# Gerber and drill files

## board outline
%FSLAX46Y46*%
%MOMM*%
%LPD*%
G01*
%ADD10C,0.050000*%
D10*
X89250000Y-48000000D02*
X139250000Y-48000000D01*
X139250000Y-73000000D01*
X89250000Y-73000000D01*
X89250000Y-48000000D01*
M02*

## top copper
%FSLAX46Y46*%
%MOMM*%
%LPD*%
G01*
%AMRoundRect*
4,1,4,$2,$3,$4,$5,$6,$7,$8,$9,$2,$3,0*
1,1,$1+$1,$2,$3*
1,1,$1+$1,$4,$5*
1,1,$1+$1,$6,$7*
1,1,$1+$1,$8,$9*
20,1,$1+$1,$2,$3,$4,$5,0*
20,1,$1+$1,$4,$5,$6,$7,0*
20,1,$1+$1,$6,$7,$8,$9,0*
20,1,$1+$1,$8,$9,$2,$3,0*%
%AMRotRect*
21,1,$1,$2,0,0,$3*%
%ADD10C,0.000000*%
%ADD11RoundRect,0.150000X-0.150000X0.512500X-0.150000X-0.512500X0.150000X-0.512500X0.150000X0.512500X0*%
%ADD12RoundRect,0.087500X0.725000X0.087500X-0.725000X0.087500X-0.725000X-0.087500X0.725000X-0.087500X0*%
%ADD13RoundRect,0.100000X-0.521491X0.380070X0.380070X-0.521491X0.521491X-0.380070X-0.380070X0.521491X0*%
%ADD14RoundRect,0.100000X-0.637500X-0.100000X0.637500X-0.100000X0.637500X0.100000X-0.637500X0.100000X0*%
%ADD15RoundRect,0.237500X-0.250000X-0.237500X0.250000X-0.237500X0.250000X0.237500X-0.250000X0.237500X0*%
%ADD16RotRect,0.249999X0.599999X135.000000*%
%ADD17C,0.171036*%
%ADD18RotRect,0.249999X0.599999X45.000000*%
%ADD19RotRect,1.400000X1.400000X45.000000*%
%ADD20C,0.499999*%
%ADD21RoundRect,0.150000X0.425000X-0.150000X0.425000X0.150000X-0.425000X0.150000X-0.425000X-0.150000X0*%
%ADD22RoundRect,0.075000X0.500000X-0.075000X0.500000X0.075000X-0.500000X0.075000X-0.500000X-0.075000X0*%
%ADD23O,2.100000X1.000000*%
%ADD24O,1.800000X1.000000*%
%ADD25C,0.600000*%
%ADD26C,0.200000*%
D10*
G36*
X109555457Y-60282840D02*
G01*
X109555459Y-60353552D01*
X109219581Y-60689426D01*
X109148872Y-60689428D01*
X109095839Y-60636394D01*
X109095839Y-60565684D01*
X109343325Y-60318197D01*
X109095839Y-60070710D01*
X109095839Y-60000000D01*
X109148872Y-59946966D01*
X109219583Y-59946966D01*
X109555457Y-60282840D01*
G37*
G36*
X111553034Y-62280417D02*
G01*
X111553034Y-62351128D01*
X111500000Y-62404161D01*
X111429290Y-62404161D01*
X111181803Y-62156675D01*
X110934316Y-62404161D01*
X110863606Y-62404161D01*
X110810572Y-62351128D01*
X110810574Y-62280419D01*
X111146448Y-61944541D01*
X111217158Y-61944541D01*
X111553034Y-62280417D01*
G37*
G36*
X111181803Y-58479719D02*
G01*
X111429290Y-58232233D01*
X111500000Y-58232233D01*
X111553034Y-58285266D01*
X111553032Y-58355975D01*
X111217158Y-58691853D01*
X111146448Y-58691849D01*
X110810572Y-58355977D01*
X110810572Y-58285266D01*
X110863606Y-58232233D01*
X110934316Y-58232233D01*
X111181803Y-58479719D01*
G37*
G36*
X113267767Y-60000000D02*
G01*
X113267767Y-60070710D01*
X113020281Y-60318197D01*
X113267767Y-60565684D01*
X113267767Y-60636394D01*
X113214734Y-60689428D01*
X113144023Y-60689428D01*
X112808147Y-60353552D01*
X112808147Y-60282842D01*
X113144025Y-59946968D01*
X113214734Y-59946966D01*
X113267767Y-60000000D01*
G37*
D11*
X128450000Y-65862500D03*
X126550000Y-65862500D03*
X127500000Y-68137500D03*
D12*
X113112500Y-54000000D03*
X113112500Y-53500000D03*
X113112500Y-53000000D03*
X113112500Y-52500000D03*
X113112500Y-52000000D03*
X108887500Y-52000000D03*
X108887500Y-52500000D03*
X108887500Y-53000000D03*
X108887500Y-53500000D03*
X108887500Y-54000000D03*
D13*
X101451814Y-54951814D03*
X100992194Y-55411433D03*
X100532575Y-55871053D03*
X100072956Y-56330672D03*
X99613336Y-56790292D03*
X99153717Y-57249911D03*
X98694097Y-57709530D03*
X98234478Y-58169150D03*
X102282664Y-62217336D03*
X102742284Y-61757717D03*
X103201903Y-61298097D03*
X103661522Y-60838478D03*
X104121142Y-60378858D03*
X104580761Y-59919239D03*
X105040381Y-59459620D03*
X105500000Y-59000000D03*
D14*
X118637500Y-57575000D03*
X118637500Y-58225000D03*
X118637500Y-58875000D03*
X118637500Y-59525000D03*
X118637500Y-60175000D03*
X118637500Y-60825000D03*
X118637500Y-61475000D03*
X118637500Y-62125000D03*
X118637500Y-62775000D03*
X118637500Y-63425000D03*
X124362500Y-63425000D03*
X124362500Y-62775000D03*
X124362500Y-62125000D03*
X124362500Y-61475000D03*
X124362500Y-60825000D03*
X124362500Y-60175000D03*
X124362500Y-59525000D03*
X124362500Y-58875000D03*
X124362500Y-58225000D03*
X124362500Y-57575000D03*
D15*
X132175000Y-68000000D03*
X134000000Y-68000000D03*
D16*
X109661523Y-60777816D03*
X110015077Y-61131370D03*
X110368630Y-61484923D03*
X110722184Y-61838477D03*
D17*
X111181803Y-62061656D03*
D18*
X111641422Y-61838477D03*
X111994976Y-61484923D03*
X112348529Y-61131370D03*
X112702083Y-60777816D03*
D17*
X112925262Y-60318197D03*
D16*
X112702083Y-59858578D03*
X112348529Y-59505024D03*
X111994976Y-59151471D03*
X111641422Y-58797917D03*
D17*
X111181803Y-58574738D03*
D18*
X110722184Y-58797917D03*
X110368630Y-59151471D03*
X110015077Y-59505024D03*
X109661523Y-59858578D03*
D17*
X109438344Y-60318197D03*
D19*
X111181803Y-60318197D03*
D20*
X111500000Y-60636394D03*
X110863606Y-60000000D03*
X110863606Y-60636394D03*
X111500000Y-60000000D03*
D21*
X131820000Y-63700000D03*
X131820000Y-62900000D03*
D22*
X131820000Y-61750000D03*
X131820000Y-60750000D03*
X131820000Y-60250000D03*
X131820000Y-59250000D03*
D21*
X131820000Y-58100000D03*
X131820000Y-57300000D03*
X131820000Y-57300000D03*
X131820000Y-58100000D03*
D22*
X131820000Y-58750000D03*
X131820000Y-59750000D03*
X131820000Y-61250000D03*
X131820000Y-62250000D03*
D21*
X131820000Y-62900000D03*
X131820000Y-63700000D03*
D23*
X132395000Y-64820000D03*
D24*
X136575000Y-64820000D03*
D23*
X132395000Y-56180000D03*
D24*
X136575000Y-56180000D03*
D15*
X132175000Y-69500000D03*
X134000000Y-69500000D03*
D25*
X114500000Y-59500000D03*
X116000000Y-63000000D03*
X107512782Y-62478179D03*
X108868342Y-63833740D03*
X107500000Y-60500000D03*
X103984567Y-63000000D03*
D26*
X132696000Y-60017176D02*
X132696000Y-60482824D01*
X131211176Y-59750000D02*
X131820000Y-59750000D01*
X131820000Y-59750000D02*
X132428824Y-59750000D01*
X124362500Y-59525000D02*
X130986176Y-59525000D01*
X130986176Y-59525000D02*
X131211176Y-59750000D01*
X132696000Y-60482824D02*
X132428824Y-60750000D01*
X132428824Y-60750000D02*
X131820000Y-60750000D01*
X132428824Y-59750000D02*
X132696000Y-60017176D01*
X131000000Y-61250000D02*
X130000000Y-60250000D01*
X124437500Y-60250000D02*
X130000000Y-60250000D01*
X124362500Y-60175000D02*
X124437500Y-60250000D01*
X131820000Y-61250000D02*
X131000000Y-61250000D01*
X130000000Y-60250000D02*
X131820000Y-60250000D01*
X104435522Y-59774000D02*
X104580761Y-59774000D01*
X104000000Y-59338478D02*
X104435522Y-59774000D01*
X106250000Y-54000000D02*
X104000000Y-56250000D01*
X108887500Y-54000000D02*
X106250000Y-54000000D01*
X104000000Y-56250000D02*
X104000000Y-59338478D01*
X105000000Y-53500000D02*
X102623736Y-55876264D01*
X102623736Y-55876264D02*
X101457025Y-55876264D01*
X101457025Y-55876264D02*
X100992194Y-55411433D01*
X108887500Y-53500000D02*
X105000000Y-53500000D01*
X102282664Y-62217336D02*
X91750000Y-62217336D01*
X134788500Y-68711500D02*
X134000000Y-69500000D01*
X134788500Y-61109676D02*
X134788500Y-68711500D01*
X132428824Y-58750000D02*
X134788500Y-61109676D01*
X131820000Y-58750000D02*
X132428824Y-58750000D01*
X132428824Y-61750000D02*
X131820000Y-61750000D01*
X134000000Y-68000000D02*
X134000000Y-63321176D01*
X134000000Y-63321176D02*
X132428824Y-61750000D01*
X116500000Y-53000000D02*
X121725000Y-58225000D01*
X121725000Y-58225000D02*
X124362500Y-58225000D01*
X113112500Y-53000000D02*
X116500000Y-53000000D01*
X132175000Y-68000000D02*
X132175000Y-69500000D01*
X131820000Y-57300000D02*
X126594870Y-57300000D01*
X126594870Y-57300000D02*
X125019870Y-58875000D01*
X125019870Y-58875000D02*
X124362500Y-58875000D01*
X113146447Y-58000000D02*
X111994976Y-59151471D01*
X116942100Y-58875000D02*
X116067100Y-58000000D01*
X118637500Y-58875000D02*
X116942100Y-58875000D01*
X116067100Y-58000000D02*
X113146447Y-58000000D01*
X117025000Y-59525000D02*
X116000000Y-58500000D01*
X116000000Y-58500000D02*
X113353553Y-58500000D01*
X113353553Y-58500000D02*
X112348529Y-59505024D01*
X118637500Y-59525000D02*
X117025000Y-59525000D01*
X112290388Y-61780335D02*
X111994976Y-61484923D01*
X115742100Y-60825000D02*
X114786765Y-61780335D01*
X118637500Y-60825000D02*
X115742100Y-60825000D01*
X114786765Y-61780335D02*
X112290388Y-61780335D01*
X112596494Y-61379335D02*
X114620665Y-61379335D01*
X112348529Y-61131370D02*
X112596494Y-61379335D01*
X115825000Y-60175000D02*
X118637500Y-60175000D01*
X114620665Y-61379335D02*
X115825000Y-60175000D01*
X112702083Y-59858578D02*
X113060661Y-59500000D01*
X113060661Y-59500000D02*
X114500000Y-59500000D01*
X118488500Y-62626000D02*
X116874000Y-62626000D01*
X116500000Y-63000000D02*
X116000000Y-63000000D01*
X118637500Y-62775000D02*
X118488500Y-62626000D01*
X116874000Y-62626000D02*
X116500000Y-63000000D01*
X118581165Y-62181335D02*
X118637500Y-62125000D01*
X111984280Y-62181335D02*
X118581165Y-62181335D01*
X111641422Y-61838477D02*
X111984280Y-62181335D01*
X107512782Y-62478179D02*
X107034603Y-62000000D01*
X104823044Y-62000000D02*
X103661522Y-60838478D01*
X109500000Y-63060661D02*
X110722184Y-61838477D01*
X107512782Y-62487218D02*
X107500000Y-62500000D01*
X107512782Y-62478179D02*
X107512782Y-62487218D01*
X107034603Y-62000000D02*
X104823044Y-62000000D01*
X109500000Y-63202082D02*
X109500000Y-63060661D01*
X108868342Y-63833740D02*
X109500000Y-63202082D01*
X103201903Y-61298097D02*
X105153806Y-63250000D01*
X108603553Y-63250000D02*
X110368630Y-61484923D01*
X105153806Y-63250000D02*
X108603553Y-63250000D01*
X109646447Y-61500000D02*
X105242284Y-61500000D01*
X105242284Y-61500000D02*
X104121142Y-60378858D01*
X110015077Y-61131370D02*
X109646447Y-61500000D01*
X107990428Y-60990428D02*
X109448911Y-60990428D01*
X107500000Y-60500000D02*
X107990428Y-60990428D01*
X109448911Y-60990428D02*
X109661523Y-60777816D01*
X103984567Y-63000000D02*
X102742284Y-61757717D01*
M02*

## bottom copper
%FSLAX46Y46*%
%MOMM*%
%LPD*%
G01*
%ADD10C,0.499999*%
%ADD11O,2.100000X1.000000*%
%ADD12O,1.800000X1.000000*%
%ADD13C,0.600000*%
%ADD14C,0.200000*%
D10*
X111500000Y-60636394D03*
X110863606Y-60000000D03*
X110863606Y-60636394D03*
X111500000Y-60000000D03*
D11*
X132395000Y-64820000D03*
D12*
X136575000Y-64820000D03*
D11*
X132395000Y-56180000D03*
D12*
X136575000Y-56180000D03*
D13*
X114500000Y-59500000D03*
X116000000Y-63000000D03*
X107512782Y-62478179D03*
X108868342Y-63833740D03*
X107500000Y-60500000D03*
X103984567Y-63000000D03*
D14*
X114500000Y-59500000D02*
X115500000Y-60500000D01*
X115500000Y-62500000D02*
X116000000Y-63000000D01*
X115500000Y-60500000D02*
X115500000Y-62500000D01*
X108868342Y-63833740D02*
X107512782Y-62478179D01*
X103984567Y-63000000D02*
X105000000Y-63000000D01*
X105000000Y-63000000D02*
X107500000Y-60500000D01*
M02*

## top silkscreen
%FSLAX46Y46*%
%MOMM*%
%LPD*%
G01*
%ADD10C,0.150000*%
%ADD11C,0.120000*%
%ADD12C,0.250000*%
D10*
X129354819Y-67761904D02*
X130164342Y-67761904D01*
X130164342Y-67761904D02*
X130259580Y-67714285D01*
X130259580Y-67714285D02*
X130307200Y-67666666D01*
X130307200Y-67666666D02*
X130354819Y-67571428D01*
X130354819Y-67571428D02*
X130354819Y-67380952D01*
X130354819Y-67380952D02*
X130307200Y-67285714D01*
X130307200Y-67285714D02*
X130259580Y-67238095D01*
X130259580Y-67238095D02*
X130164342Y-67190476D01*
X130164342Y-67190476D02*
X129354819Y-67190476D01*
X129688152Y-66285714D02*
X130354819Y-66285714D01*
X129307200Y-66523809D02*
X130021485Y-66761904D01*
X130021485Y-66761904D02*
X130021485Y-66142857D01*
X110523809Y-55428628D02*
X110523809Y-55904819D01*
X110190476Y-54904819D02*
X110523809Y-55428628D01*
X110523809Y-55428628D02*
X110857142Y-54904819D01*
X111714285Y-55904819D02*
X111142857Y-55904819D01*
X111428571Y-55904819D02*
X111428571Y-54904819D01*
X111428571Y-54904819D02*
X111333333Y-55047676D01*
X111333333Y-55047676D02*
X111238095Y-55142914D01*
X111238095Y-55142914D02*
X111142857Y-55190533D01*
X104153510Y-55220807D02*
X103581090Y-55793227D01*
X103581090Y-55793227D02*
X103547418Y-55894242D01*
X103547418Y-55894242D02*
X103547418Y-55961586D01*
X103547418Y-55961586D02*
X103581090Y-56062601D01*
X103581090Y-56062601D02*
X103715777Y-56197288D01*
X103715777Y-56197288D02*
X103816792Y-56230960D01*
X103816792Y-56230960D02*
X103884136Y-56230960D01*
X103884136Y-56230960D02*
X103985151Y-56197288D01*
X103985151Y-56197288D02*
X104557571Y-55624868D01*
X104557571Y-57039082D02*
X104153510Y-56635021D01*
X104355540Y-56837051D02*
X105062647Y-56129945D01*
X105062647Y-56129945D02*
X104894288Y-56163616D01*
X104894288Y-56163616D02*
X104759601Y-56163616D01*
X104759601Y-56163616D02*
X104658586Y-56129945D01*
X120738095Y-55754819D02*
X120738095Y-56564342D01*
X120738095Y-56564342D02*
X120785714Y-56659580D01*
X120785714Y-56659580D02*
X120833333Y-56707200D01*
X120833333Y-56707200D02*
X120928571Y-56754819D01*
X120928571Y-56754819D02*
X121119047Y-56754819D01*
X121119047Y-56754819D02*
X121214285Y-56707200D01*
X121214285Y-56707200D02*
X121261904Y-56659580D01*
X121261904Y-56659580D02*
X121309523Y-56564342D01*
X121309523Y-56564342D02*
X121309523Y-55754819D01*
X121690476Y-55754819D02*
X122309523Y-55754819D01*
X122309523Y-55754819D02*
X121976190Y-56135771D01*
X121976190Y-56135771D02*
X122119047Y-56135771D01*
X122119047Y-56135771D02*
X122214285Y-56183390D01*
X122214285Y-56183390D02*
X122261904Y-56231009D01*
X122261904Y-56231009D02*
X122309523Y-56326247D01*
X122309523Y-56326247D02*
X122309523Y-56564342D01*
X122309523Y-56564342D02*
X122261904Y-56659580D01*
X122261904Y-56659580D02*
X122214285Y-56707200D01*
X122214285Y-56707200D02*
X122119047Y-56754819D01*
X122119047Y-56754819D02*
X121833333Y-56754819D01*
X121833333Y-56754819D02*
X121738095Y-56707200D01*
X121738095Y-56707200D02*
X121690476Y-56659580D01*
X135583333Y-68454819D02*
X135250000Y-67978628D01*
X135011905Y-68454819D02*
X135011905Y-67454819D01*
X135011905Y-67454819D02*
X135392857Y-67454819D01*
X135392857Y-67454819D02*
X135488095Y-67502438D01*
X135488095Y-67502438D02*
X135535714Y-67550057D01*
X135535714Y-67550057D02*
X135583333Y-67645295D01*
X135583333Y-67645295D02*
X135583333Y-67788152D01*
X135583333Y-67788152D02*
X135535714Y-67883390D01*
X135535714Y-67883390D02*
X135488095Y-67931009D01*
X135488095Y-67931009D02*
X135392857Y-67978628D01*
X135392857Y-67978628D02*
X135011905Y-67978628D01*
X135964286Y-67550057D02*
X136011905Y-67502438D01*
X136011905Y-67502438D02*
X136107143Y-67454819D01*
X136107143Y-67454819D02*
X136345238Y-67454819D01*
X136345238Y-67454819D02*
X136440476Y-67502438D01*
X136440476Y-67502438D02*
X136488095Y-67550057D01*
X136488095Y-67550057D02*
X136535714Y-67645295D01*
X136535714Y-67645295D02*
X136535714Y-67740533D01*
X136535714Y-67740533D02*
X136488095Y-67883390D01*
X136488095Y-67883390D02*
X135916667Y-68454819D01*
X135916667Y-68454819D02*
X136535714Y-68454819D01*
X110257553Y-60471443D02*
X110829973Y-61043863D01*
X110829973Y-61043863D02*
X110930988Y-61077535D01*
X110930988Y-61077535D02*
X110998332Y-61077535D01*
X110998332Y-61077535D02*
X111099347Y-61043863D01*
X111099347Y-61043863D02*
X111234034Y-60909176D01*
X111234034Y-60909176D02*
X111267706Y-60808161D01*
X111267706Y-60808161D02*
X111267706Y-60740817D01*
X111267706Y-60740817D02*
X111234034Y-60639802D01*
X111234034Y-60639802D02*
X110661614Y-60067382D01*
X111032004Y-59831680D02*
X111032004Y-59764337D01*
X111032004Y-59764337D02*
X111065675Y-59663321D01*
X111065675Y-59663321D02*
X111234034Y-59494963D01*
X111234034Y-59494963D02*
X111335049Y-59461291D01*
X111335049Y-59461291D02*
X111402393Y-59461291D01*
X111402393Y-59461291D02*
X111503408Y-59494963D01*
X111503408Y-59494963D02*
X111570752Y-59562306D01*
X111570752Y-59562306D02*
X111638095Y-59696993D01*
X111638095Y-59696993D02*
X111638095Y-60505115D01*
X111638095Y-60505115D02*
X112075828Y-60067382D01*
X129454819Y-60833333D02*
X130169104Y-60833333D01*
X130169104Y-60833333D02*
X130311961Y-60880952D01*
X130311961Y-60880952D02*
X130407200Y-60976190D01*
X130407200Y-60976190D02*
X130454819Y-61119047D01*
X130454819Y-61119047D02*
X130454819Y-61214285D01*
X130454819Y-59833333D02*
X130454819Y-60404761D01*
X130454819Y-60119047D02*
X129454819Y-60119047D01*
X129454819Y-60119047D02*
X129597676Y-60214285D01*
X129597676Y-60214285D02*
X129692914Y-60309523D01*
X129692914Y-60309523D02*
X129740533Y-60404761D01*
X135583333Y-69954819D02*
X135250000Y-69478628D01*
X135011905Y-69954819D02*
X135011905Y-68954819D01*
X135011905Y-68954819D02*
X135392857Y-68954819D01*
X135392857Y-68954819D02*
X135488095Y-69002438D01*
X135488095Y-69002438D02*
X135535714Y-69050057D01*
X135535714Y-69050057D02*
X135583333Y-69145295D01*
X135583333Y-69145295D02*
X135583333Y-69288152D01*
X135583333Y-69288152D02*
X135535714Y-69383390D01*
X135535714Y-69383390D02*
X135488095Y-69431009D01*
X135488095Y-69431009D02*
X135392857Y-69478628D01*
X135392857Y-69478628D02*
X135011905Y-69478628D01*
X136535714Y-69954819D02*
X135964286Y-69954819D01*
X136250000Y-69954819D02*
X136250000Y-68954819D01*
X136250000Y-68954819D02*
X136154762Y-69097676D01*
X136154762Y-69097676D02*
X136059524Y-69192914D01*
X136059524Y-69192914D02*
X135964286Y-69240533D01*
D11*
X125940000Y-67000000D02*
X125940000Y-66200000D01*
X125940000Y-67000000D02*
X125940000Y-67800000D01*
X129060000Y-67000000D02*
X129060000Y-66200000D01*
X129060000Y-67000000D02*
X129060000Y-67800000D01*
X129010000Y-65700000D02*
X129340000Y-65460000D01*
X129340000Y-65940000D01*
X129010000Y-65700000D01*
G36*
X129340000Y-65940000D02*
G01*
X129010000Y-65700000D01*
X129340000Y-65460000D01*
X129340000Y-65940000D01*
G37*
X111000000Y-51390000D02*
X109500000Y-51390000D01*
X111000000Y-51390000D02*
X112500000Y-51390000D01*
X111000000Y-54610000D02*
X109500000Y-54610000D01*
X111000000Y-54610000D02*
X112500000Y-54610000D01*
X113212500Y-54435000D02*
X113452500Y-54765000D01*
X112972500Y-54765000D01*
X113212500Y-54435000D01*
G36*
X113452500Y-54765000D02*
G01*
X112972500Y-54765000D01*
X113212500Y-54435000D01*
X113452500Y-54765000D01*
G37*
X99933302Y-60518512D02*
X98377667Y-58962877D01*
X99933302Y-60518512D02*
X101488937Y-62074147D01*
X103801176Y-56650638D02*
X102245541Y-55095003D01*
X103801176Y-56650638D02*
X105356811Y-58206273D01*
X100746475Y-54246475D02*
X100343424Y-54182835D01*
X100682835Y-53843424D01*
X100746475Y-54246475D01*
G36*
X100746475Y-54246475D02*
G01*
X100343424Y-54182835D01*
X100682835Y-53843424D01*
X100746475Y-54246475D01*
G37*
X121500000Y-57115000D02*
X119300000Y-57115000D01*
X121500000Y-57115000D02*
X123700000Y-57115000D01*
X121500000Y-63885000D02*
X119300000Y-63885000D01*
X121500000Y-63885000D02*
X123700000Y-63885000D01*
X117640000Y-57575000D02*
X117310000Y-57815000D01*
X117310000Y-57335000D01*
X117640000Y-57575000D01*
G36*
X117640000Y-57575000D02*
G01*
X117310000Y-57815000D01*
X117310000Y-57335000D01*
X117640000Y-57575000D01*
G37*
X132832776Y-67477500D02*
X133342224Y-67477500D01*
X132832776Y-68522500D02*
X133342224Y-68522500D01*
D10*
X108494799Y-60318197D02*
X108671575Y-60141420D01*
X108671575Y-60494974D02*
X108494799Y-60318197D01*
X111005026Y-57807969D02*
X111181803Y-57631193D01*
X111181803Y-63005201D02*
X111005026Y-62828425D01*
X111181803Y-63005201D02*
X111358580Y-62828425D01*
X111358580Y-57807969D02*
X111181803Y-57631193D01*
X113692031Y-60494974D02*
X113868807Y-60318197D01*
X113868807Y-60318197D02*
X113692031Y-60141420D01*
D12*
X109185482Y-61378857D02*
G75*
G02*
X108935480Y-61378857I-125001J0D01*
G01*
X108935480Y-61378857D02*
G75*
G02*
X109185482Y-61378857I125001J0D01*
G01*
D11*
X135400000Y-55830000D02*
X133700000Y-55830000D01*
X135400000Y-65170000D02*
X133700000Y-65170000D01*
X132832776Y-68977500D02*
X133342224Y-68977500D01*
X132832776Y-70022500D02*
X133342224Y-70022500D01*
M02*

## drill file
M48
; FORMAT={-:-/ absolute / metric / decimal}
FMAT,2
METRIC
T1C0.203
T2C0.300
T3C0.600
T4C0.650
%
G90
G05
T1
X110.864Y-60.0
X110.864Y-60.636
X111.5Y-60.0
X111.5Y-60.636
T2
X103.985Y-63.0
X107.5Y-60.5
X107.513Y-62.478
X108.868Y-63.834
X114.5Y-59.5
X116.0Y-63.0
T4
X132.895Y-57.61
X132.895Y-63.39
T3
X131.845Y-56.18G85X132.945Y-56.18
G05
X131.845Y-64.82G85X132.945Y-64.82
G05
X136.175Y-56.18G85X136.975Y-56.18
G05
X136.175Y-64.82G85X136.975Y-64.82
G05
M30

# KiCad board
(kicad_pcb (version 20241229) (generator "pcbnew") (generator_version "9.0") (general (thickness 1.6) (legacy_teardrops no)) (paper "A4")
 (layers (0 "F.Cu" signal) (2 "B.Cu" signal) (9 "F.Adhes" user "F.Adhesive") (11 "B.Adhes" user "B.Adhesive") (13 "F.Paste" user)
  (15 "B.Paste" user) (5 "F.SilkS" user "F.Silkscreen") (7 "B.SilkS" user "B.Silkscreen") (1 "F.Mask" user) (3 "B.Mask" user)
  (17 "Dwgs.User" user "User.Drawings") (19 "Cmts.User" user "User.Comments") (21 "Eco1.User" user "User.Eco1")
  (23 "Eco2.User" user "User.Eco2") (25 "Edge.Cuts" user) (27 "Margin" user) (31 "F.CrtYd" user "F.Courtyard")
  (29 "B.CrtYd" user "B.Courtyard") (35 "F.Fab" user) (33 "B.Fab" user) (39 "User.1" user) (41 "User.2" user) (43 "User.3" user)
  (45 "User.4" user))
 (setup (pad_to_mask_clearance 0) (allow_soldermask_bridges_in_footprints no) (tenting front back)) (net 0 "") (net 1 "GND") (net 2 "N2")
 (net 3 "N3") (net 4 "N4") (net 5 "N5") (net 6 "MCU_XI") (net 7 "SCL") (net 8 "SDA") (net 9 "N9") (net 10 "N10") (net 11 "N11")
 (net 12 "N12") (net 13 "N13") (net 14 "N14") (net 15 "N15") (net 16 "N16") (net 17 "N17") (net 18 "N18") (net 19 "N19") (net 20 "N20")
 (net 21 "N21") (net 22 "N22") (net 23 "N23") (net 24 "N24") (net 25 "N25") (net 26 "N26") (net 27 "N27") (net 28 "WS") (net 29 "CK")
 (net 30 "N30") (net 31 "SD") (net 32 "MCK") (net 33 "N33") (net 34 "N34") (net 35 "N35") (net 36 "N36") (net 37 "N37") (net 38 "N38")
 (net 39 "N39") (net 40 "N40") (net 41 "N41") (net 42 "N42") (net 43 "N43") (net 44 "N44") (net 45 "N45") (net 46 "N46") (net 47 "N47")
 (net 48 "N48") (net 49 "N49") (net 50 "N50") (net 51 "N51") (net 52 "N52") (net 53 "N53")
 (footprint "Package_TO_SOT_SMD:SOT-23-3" (layer "F.Cu") (at 127.5 67 -90)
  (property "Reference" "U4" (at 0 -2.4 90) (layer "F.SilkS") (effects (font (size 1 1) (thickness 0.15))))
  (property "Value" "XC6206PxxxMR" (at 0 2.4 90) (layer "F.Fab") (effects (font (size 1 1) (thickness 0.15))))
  (fp_line (start 0 1.56) (end -0.8 1.56) (stroke (width 0.12) (type solid)) (layer "F.SilkS"))
  (fp_line (start 0 1.56) (end 0.8 1.56) (stroke (width 0.12) (type solid)) (layer "F.SilkS"))
  (fp_line (start 0 -1.56) (end -0.8 -1.56) (stroke (width 0.12) (type solid)) (layer "F.SilkS"))
  (fp_line (start 0 -1.56) (end 0.8 -1.56) (stroke (width 0.12) (type solid)) (layer "F.SilkS"))
  (fp_poly (pts (xy -1.3 -1.51) (xy -1.54 -1.84) (xy -1.06 -1.84)) (stroke (width 0.12) (type solid)) (fill yes) (layer "F.SilkS"))
  (pad "1" smd roundrect (at -1.1375 -0.95 270) (size 1.325 0.6) (layers "F.Cu" "F.Mask" "F.Paste") (roundrect_rratio 0.25) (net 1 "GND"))
  (pad "2" smd roundrect (at -1.1375 0.95 270) (size 1.325 0.6) (layers "F.Cu" "F.Mask" "F.Paste") (roundrect_rratio 0.25) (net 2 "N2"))
  (pad "3" smd roundrect (at 1.1375 0 270) (size 1.325 0.6) (layers "F.Cu" "F.Mask" "F.Paste") (roundrect_rratio 0.25) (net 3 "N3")))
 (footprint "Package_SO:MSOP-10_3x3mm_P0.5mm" (layer "F.Cu") (at 111 53 180)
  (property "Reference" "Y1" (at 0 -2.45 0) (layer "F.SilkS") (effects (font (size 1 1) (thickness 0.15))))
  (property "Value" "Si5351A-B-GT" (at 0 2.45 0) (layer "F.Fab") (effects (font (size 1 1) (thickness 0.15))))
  (fp_line (start 0 1.61) (end 1.5 1.61) (stroke (width 0.12) (type solid)) (layer "F.SilkS"))
  (fp_line (start 0 1.61) (end -1.5 1.61) (stroke (width 0.12) (type solid)) (layer "F.SilkS"))
  (fp_line (start 0 -1.61) (end 1.5 -1.61) (stroke (width 0.12) (type solid)) (layer "F.SilkS"))
  (fp_line (start 0 -1.61) (end -1.5 -1.61) (stroke (width 0.12) (type solid)) (layer "F.SilkS"))
  (fp_poly
   (pts (xy -2.2125 -1.435) (xy -2.4525 -1.765) (xy -1.9725 -1.765)) (stroke (width 0.12) (type solid)) (fill yes) (layer "F.SilkS"))
  (pad "1" smd roundrect (at -2.1125 -1 180) (size 1.625 0.35) (layers "F.Cu" "F.Mask" "F.Paste") (roundrect_rratio 0.25) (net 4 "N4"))
  (pad "2" smd roundrect (at -2.1125 -0.5 180) (size 1.625 0.35) (layers "F.Cu" "F.Mask" "F.Paste") (roundrect_rratio 0.25) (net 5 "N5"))
  (pad "3" smd roundrect (at -2.1125 0 180) (size 1.625 0.35) (layers "F.Cu" "F.Mask" "F.Paste") (roundrect_rratio 0.25) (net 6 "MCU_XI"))
  (pad "4" smd roundrect (at -2.1125 0.5 180) (size 1.625 0.35) (layers "F.Cu" "F.Mask" "F.Paste") (roundrect_rratio 0.25) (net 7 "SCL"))
  (pad "5" smd roundrect (at -2.1125 1 180) (size 1.625 0.35) (layers "F.Cu" "F.Mask" "F.Paste") (roundrect_rratio 0.25) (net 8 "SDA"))
  (pad "6" smd roundrect (at 2.1125 1 180) (size 1.625 0.35) (layers "F.Cu" "F.Mask" "F.Paste") (roundrect_rratio 0.25) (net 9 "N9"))
  (pad "7" smd roundrect (at 2.1125 0.5 180) (size 1.625 0.35) (layers "F.Cu" "F.Mask" "F.Paste") (roundrect_rratio 0.25) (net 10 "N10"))
  (pad "8" smd roundrect (at 2.1125 0 180) (size 1.625 0.35) (layers "F.Cu" "F.Mask" "F.Paste") (roundrect_rratio 0.25) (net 1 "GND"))
  (pad "9" smd roundrect (at 2.1125 -0.5 180) (size 1.625 0.35) (layers "F.Cu" "F.Mask" "F.Paste") (roundrect_rratio 0.25) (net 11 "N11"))
  (pad "10" smd roundrect (at 2.1125 -1 180) (size 1.625 0.35) (layers "F.Cu" "F.Mask" "F.Paste") (roundrect_rratio 0.25) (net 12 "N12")))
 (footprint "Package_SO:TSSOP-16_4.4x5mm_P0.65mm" (layer "F.Cu") (at 101.867239 58.584575 -45)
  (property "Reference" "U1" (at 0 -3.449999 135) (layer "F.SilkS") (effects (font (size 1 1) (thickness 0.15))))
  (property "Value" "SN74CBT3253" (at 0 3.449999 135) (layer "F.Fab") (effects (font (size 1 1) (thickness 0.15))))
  (fp_line (start 0 2.735) (end -2.2 2.735) (stroke (width 0.12) (type solid)) (layer "F.SilkS"))
  (fp_line (start 0 2.735) (end 2.2 2.735) (stroke (width 0.12) (type solid)) (layer "F.SilkS"))
  (fp_line (start 0 -2.735) (end -2.2 -2.735) (stroke (width 0.12) (type solid)) (layer "F.SilkS"))
  (fp_line (start 0 -2.735) (end 2.2 -2.735) (stroke (width 0.12) (type solid)) (layer "F.SilkS"))
  (fp_poly (pts (xy -3.86 -2.275) (xy -4.19 -2.035) (xy -4.19 -2.515)) (stroke (width 0.12) (type solid)) (fill yes) (layer "F.SilkS"))
  (pad "1" smd roundrect (at -2.8625 -2.275 315) (size 1.475 0.4) (layers "F.Cu" "F.Mask" "F.Paste") (roundrect_rratio 0.25) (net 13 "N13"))
  (pad "2" smd roundrect (at -2.8625 -1.625 315) (size 1.475 0.4) (layers "F.Cu" "F.Mask" "F.Paste") (roundrect_rratio 0.25) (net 11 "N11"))
  (pad "3" smd roundrect (at -2.8625 -0.975 315) (size 1.475 0.4) (layers "F.Cu" "F.Mask" "F.Paste") (roundrect_rratio 0.25) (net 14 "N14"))
  (pad "4" smd roundrect (at -2.8625 -0.325 315) (size 1.475 0.4) (layers "F.Cu" "F.Mask" "F.Paste") (roundrect_rratio 0.25) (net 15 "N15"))
  (pad "5" smd roundrect (at -2.8625 0.325 315) (size 1.475 0.4) (layers "F.Cu" "F.Mask" "F.Paste") (roundrect_rratio 0.25) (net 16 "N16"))
  (pad "6" smd roundrect (at -2.8625 0.975 315) (size 1.475 0.4) (layers "F.Cu" "F.Mask" "F.Paste") (roundrect_rratio 0.25) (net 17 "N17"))
  (pad "7" smd roundrect (at -2.8625 1.625 315) (size 1.475 0.4) (layers "F.Cu" "F.Mask" "F.Paste") (roundrect_rratio 0.25) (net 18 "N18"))
  (pad "8" smd roundrect (at -2.8625 2.275 315) (size 1.475 0.4) (layers "F.Cu" "F.Mask" "F.Paste") (roundrect_rratio 0.25) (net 1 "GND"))
  (pad "9" smd roundrect (at 2.8625 2.275 315) (size 1.475 0.4) (layers "F.Cu" "F.Mask" "F.Paste") (roundrect_rratio 0.25) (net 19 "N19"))
  (pad "10" smd roundrect (at 2.8625 1.625 315) (size 1.475 0.4) (layers "F.Cu" "F.Mask" "F.Paste") (roundrect_rratio 0.25) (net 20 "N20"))
  (pad "11" smd roundrect (at 2.8625 0.975 315) (size 1.475 0.4) (layers "F.Cu" "F.Mask" "F.Paste") (roundrect_rratio 0.25) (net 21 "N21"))
  (pad "12" smd roundrect (at 2.8625 0.325 315) (size 1.475 0.4) (layers "F.Cu" "F.Mask" "F.Paste") (roundrect_rratio 0.25) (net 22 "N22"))
  (pad "13" smd roundrect (at 2.8625 -0.325 315) (size 1.475 0.4) (layers "F.Cu" "F.Mask" "F.Paste") (roundrect_rratio 0.25) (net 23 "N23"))
  (pad "14" smd roundrect (at 2.8625 -0.975 315) (size 1.475 0.4) (layers "F.Cu" "F.Mask" "F.Paste") (roundrect_rratio 0.25) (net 12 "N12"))
  (pad "15" smd roundrect (at 2.8625 -1.625 315) (size 1.475 0.4) (layers "F.Cu" "F.Mask" "F.Paste") (roundrect_rratio 0.25) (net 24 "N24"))
  (pad "16" smd roundrect (at 2.8625 -2.275 315) (size 1.475 0.4) (layers "F.Cu" "F.Mask" "F.Paste") (roundrect_rratio 0.25) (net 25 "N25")))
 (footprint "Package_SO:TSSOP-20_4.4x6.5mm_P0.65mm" (layer "F.Cu") (at 121.5 60.5)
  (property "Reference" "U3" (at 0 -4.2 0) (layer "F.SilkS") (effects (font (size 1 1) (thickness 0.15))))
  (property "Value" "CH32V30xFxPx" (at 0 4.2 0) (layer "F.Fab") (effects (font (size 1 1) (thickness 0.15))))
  (fp_line (start 0 -3.385) (end -2.2 -3.385) (stroke (width 0.12) (type solid)) (layer "F.SilkS"))
  (fp_line (start 0 -3.385) (end 2.2 -3.385) (stroke (width 0.12) (type solid)) (layer "F.SilkS"))
  (fp_line (start 0 3.385) (end -2.2 3.385) (stroke (width 0.12) (type solid)) (layer "F.SilkS"))
  (fp_line (start 0 3.385) (end 2.2 3.385) (stroke (width 0.12) (type solid)) (layer "F.SilkS"))
  (fp_poly (pts (xy -3.86 -2.925) (xy -4.19 -2.685) (xy -4.19 -3.165)) (stroke (width 0.12) (type solid)) (fill yes) (layer "F.SilkS"))
  (pad "1" smd roundrect (at -2.8625 -2.925) (size 1.475 0.4) (layers "F.Cu" "F.Mask" "F.Paste") (roundrect_rratio 0.25) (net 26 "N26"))
  (pad "2" smd roundrect (at -2.8625 -2.275) (size 1.475 0.4) (layers "F.Cu" "F.Mask" "F.Paste") (roundrect_rratio 0.25) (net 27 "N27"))
  (pad "3" smd roundrect (at -2.8625 -1.625) (size 1.475 0.4) (layers "F.Cu" "F.Mask" "F.Paste") (roundrect_rratio 0.25) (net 7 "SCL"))
  (pad "4" smd roundrect (at -2.8625 -0.975) (size 1.475 0.4) (layers "F.Cu" "F.Mask" "F.Paste") (roundrect_rratio 0.25) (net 8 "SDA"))
  (pad "5" smd roundrect (at -2.8625 -0.325) (size 1.475 0.4) (layers "F.Cu" "F.Mask" "F.Paste") (roundrect_rratio 0.25) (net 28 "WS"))
  (pad "6" smd roundrect (at -2.8625 0.325) (size 1.475 0.4) (layers "F.Cu" "F.Mask" "F.Paste") (roundrect_rratio 0.25) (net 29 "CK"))
  (pad "7" smd roundrect (at -2.8625 0.975) (size 1.475 0.4) (layers "F.Cu" "F.Mask" "F.Paste") (roundrect_rratio 0.25) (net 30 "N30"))
  (pad "8" smd roundrect (at -2.8625 1.625) (size 1.475 0.4) (layers "F.Cu" "F.Mask" "F.Paste") (roundrect_rratio 0.25) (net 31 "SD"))
  (pad "9" smd roundrect (at -2.8625 2.275) (size 1.475 0.4) (layers "F.Cu" "F.Mask" "F.Paste") (roundrect_rratio 0.25) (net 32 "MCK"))
  (pad "10" smd roundrect (at -2.8625 2.925) (size 1.475 0.4) (layers "F.Cu" "F.Mask" "F.Paste") (roundrect_rratio 0.25) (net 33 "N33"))
  (pad "11" smd roundrect (at 2.8625 2.925) (size 1.475 0.4) (layers "F.Cu" "F.Mask" "F.Paste") (roundrect_rratio 0.25) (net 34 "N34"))
  (pad "12" smd roundrect (at 2.8625 2.275) (size 1.475 0.4) (layers "F.Cu" "F.Mask" "F.Paste") (roundrect_rratio 0.25) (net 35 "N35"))
  (pad "13" smd roundrect (at 2.8625 1.625) (size 1.475 0.4) (layers "F.Cu" "F.Mask" "F.Paste") (roundrect_rratio 0.25) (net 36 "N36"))
  (pad "14" smd roundrect (at 2.8625 0.975) (size 1.475 0.4) (layers "F.Cu" "F.Mask" "F.Paste") (roundrect_rratio 0.25) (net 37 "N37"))
  (pad "15" smd roundrect (at 2.8625 0.325) (size 1.475 0.4) (layers "F.Cu" "F.Mask" "F.Paste") (roundrect_rratio 0.25) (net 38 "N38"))
  (pad "16" smd roundrect (at 2.8625 -0.325) (size 1.475 0.4) (layers "F.Cu" "F.Mask" "F.Paste") (roundrect_rratio 0.25) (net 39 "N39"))
  (pad "17" smd roundrect (at 2.8625 -0.975) (size 1.475 0.4) (layers "F.Cu" "F.Mask" "F.Paste") (roundrect_rratio 0.25) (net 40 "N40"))
  (pad "18" smd roundrect (at 2.8625 -1.625) (size 1.475 0.4) (layers "F.Cu" "F.Mask" "F.Paste") (roundrect_rratio 0.25) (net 1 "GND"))
  (pad "19" smd roundrect (at 2.8625 -2.275) (size 1.475 0.4) (layers "F.Cu" "F.Mask" "F.Paste") (roundrect_rratio 0.25) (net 6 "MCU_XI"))
  (pad "20" smd roundrect (at 2.8625 -2.925) (size 1.475 0.4) (layers "F.Cu" "F.Mask" "F.Paste") (roundrect_rratio 0.25) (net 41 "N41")))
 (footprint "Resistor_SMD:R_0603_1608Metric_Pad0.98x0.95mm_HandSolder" (layer "F.Cu") (at 133.0875 68)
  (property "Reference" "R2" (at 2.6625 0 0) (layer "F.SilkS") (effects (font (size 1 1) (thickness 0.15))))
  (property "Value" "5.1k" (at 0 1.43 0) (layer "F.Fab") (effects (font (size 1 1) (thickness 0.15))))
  (fp_line (start -0.254724 -0.5225) (end 0.254724 -0.5225) (stroke (width 0.12) (type solid)) (layer "F.SilkS"))
  (fp_line (start -0.254724 0.5225) (end 0.254724 0.5225) (stroke (width 0.12) (type solid)) (layer "F.SilkS"))
  (pad "1" smd roundrect (at -0.9125 0) (size 0.975 0.95) (layers "F.Cu" "F.Mask" "F.Paste") (roundrect_rratio 0.25) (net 1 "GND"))
  (pad "2" smd roundrect (at 0.9125 0) (size 0.975 0.95) (layers "F.Cu" "F.Mask" "F.Paste") (roundrect_rratio 0.25) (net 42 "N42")))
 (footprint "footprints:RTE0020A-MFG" (layer "F.Cu") (at 111.181803 60.318197 45)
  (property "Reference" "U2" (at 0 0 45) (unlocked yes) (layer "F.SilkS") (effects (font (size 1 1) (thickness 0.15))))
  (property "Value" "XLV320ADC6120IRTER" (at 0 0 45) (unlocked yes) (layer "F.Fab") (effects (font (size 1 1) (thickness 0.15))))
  (fp_poly
   (pts (xy -1.649999 -1.125002) (xy -1.699999 -1.174999) (xy -1.699999 -1.25) (xy -1.649999 -1.3) (xy -1.3 -1.3) (xy -1.3 -1.649999)
    (xy -1.25 -1.699999) (xy -1.174999 -1.699999) (xy -1.124999 -1.649999) (xy -1.124999 -1.175001) (xy -1.174999 -1.124999))
   (stroke (width 0) (type solid)) (fill yes) (layer "F.Cu"))
  (fp_poly
   (pts (xy -1.649999 1.125002) (xy -1.699999 1.174999) (xy -1.699999 1.25) (xy -1.649999 1.3) (xy -1.3 1.3) (xy -1.3 1.649999)
    (xy -1.25 1.699999) (xy -1.174999 1.699999) (xy -1.124999 1.649999) (xy -1.124999 1.174999) (xy -1.174999 1.124999))
   (stroke (width 0) (type solid)) (fill yes) (layer "F.Cu"))
  (fp_poly
   (pts (xy 1.649999 -1.125002) (xy 1.699999 -1.174999) (xy 1.699999 -1.25) (xy 1.649999 -1.3) (xy 1.3 -1.3) (xy 1.3 -1.649999)
    (xy 1.25 -1.699999) (xy 1.174999 -1.699999) (xy 1.124999 -1.649999) (xy 1.125002 -1.175001) (xy 1.174999 -1.124999))
   (stroke (width 0) (type solid)) (fill yes) (layer "F.Cu"))
  (fp_poly
   (pts (xy 1.649999 1.125002) (xy 1.699999 1.174999) (xy 1.699999 1.25) (xy 1.649999 1.3) (xy 1.3 1.3) (xy 1.3 1.649999) (xy 1.25 1.699999)
    (xy 1.174999 1.699999) (xy 1.124999 1.649999) (xy 1.124999 1.174999) (xy 1.174999 1.124999))
   (stroke (width 0) (type solid)) (fill yes) (layer "F.Cu"))
  (fp_line (start -1.899999 -1.899999) (end -1.649999 -1.899999) (stroke (width 0.15) (type solid)) (layer "F.SilkS"))
  (fp_line (start -1.899999 -1.649999) (end -1.899999 -1.899999) (stroke (width 0.15) (type solid)) (layer "F.SilkS"))
  (fp_line (start 1.649999 -1.899999) (end 1.899999 -1.899999) (stroke (width 0.15) (type solid)) (layer "F.SilkS"))
  (fp_line (start -1.899999 1.899999) (end -1.899999 1.649999) (stroke (width 0.15) (type solid)) (layer "F.SilkS"))
  (fp_line (start -1.899999 1.899999) (end -1.649999 1.899999) (stroke (width 0.15) (type solid)) (layer "F.SilkS"))
  (fp_line (start 1.899999 -1.649999) (end 1.899999 -1.899999) (stroke (width 0.15) (type solid)) (layer "F.SilkS"))
  (fp_line (start 1.649999 1.899999) (end 1.899999 1.899999) (stroke (width 0.15) (type solid)) (layer "F.SilkS"))
  (fp_line (start 1.899999 1.899999) (end 1.899999 1.649999) (stroke (width 0.15) (type solid)) (layer "F.SilkS"))
  (fp_circle (center -2.250001 -0.750001) (end -2.125 -0.750001) (stroke (width 0.25) (type solid)) (fill no) (layer "F.SilkS"))
  (pad "1" smd rect (at -1.4 -0.750001 135) (size 0.249999 0.599999) (layers "F.Cu" "F.Mask" "F.Paste") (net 20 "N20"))
  (pad "2" smd rect (at -1.4 -0.25 135) (size 0.249999 0.599999) (layers "F.Cu" "F.Mask" "F.Paste") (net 23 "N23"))
  (pad "3" smd rect (at -1.4 0.25 135) (size 0.249999 0.599999) (layers "F.Cu" "F.Mask" "F.Paste") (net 21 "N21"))
  (pad "4" smd rect (at -1.4 0.750001 135) (size 0.249999 0.599999) (layers "F.Cu" "F.Mask" "F.Paste") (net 22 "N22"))
  (pad "5" smd circle (at -1.232812 1.232812 45) (size 0.171036 0.171036) (layers "F.Cu" "F.Mask" "F.Paste") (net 1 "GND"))
  (pad "6" smd rect (at -0.750001 1.4 45) (size 0.249999 0.599999) (layers "F.Cu" "F.Mask" "F.Paste") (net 31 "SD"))
  (pad "7" smd rect (at -0.25 1.4 45) (size 0.249999 0.599999) (layers "F.Cu" "F.Mask" "F.Paste") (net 29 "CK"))
  (pad "8" smd rect (at 0.25 1.4 45) (size 0.249999 0.599999) (layers "F.Cu" "F.Mask" "F.Paste") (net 28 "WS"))
  (pad "9" smd rect (at 0.750001 1.4 45) (size 0.249999 0.599999) (layers "F.Cu" "F.Mask" "F.Paste") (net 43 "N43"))
  (pad "10" smd circle (at 1.232812 1.232812 45) (size 0.171036 0.171036) (layers "F.Cu" "F.Mask" "F.Paste") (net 1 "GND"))
  (pad "11" smd rect (at 1.4 0.750001 135) (size 0.249999 0.599999) (layers "F.Cu" "F.Mask" "F.Paste") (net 32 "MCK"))
  (pad "12" smd rect (at 1.4 0.25 135) (size 0.249999 0.599999) (layers "F.Cu" "F.Mask" "F.Paste") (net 8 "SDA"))
  (pad "13" smd rect (at 1.4 -0.25 135) (size 0.249999 0.599999) (layers "F.Cu" "F.Mask" "F.Paste") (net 7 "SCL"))
  (pad "14" smd rect (at 1.4 -0.750001 135) (size 0.249999 0.599999) (layers "F.Cu" "F.Mask" "F.Paste") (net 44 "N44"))
  (pad "15" smd circle (at 1.232812 -1.232812 45) (size 0.171036 0.171036) (layers "F.Cu" "F.Mask" "F.Paste") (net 1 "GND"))
  (pad "16" smd rect (at 0.750001 -1.4 45) (size 0.249999 0.599999) (layers "F.Cu" "F.Mask" "F.Paste") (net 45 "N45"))
  (pad "17" smd rect (at 0.25 -1.4 45) (size 0.249999 0.599999) (layers "F.Cu" "F.Mask" "F.Paste") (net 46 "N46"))
  (pad "18" smd rect (at -0.25 -1.4 45) (size 0.249999 0.599999) (layers "F.Cu" "F.Mask" "F.Paste") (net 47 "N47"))
  (pad "19" smd rect (at -0.750001 -1.4 45) (size 0.249999 0.599999) (layers "F.Cu" "F.Mask" "F.Paste") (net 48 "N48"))
  (pad "20" smd circle (at -1.232812 -1.232812 45) (size 0.171036 0.171036) (layers "F.Cu" "F.Mask" "F.Paste") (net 1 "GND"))
  (pad "21" smd rect (at 0 0 45) (size 1.4 1.4) (layers "F.Cu" "F.Mask") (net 1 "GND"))
  (pad "22" thru_hole circle (at 0 0.449999 45) (size 0.499999 0.499999) (drill 0.2032) (layers "*.Cu" "*.Mask") (remove_unused_layers no))
  (pad "23" thru_hole circle (at 0 -0.449999 45) (size 0.499999 0.499999) (drill 0.2032) (layers "*.Cu" "*.Mask") (remove_unused_layers no))
  (pad "24" thru_hole circle (at -0.449999 0 45) (size 0.499999 0.499999) (drill 0.2032) (layers "*.Cu" "*.Mask") (remove_unused_layers no))
  (pad "25" thru_hole circle (at 0.449999 0 45) (size 0.499999 0.499999) (drill 0.2032) (layers "*.Cu" "*.Mask") (remove_unused_layers no)))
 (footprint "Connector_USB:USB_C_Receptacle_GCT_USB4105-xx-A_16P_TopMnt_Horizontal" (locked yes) (layer "F.Cu") (at 135.5 60.5 90)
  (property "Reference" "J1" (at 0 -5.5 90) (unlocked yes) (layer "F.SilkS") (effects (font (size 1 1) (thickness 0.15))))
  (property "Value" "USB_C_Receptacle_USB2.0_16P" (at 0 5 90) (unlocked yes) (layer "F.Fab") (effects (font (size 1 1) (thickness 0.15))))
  (fp_line (start 4.67 -0.1) (end 4.67 -1.8) (stroke (width 0.12) (type solid)) (layer "F.SilkS"))
  (fp_line (start -4.67 -0.1) (end -4.67 -1.8) (stroke (width 0.12) (type solid)) (layer "F.SilkS"))
  (pad "" np_thru_hole circle (at -2.89 -2.605 90) (size 0.65 0.65) (drill 0.65) (layers "*.Cu" "*.Mask"))
  (pad "" np_thru_hole circle (at 2.89 -2.605 90) (size 0.65 0.65) (drill 0.65) (layers "*.Cu" "*.Mask"))
  (pad "A1" smd roundrect (at -3.2 -3.68 90) (size 0.6 1.15) (layers "F.Cu" "F.Mask" "F.Paste") (roundrect_rratio 0.25) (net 1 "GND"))
  (pad "A4" smd roundrect (at -2.4 -3.68 90) (size 0.6 1.15) (layers "F.Cu" "F.Mask" "F.Paste") (roundrect_rratio 0.25) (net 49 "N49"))
  (pad "A5" smd roundrect (at -1.25 -3.68 90) (size 0.3 1.15) (layers "F.Cu" "F.Mask" "F.Paste") (roundrect_rratio 0.25) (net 42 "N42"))
  (pad "A6" smd roundrect (at -0.25 -3.68 90) (size 0.3 1.15) (layers "F.Cu" "F.Mask" "F.Paste") (roundrect_rratio 0.25) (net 40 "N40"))
  (pad "A7" smd roundrect (at 0.25 -3.68 90) (size 0.3 1.15) (layers "F.Cu" "F.Mask" "F.Paste") (roundrect_rratio 0.25) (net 39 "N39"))
  (pad "A8" smd roundrect (at 1.25 -3.68 90) (size 0.3 1.15) (layers "F.Cu" "F.Mask" "F.Paste") (roundrect_rratio 0.25) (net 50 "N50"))
  (pad "A9" smd roundrect (at 2.4 -3.68 90) (size 0.6 1.15) (layers "F.Cu" "F.Mask" "F.Paste") (roundrect_rratio 0.25) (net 49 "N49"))
  (pad "A12" smd roundrect (at 3.2 -3.68 90) (size 0.6 1.15) (layers "F.Cu" "F.Mask" "F.Paste") (roundrect_rratio 0.25) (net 1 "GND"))
  (pad "B1" smd roundrect (at 3.2 -3.68 90) (size 0.6 1.15) (layers "F.Cu" "F.Mask" "F.Paste") (roundrect_rratio 0.25) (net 1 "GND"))
  (pad "B4" smd roundrect (at 2.4 -3.68 90) (size 0.6 1.15) (layers "F.Cu" "F.Mask" "F.Paste") (roundrect_rratio 0.25) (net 49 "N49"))
  (pad "B5" smd roundrect (at 1.75 -3.68 90) (size 0.3 1.15) (layers "F.Cu" "F.Mask" "F.Paste") (roundrect_rratio 0.25) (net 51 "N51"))
  (pad "B6" smd roundrect (at 0.75 -3.68 90) (size 0.3 1.15) (layers "F.Cu" "F.Mask" "F.Paste") (roundrect_rratio 0.25) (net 40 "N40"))
  (pad "B7" smd roundrect (at -0.75 -3.68 90) (size 0.3 1.15) (layers "F.Cu" "F.Mask" "F.Paste") (roundrect_rratio 0.25) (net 39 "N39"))
  (pad "B8" smd roundrect (at -1.75 -3.68 90) (size 0.3 1.15) (layers "F.Cu" "F.Mask" "F.Paste") (roundrect_rratio 0.25) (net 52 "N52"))
  (pad "B9" smd roundrect (at -2.4 -3.68 90) (size 0.6 1.15) (layers "F.Cu" "F.Mask" "F.Paste") (roundrect_rratio 0.25) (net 49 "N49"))
  (pad "B12" smd roundrect (at -3.2 -3.68 90) (size 0.6 1.15) (layers "F.Cu" "F.Mask" "F.Paste") (roundrect_rratio 0.25) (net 1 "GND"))
  (pad "S1" thru_hole oval (at -4.32 -3.105 90) (size 1 2.1) (drill oval 0.6 1.7) (layers "*.Cu" "*.Mask" "F.Paste")
   (remove_unused_layers no) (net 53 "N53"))
  (pad "S1" thru_hole oval (at -4.32 1.075 90) (size 1 1.8) (drill oval 0.6 1.4) (layers "*.Cu" "*.Mask" "F.Paste")
   (remove_unused_layers no) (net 53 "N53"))
  (pad "S1" thru_hole oval (at 4.32 -3.105 90) (size 1 2.1) (drill oval 0.6 1.7) (layers "*.Cu" "*.Mask" "F.Paste")
   (remove_unused_layers no) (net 53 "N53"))
  (pad "S1" thru_hole oval (at 4.32 1.075 90) (size 1 1.8) (drill oval 0.6 1.4) (layers "*.Cu" "*.Mask" "F.Paste") (remove_unused_layers no)
   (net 53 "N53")))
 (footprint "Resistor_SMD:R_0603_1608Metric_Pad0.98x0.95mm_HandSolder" (layer "F.Cu") (at 133.0875 69.5)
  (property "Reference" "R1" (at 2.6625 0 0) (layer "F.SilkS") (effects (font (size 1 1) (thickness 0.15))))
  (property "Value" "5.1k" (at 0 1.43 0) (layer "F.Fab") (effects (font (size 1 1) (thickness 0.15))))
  (fp_line (start -0.254724 -0.5225) (end 0.254724 -0.5225) (stroke (width 0.12) (type solid)) (layer "F.SilkS"))
  (fp_line (start -0.254724 0.5225) (end 0.254724 0.5225) (stroke (width 0.12) (type solid)) (layer "F.SilkS"))
  (pad "1" smd roundrect (at -0.9125 0) (size 0.975 0.95) (layers "F.Cu" "F.Mask" "F.Paste") (roundrect_rratio 0.25) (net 1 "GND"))
  (pad "2" smd roundrect (at 0.9125 0) (size 0.975 0.95) (layers "F.Cu" "F.Mask" "F.Paste") (roundrect_rratio 0.25) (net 51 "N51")))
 (gr_rect (start 89.25 48) (end 139.25 73) (stroke (width 0.05) (type solid)) (fill no) (layer "Edge.Cuts"))
 (segment (start 132.696 60.017176) (end 132.696 60.482824) (width 0.2) (layer "F.Cu") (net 40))
 (segment (start 131.211176 59.75) (end 131.82 59.75) (width 0.2) (layer "F.Cu") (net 40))
 (segment (start 131.82 59.75) (end 132.428824 59.75) (width 0.2) (layer "F.Cu") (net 40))
 (segment (start 124.3625 59.525) (end 130.986176 59.525) (width 0.2) (layer "F.Cu") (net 40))
 (segment (start 130.986176 59.525) (end 131.211176 59.75) (width 0.2) (layer "F.Cu") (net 40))
 (segment (start 132.696 60.482824) (end 132.428824 60.75) (width 0.2) (layer "F.Cu") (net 40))
 (segment (start 132.428824 60.75) (end 131.82 60.75) (width 0.2) (layer "F.Cu") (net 40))
 (segment (start 132.428824 59.75) (end 132.696 60.017176) (width 0.2) (layer "F.Cu") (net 40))
 (segment (start 131 61.25) (end 130 60.25) (width 0.2) (layer "F.Cu") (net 39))
 (segment (start 124.4375 60.25) (end 130 60.25) (width 0.2) (layer "F.Cu") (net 39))
 (segment (start 124.3625 60.175) (end 124.4375 60.25) (width 0.2) (layer "F.Cu") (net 39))
 (segment (start 131.82 61.25) (end 131 61.25) (width 0.2) (layer "F.Cu") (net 39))
 (segment (start 130 60.25) (end 131.82 60.25) (width 0.2) (layer "F.Cu") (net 39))
 (segment (start 104.435522 59.774) (end 104.580761 59.774) (width 0.2) (layer "F.Cu") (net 12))
 (segment (start 104 59.338478) (end 104.435522 59.774) (width 0.2) (layer "F.Cu") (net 12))
 (segment (start 106.25 54) (end 104 56.25) (width 0.2) (layer "F.Cu") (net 12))
 (segment (start 108.8875 54) (end 106.25 54) (width 0.2) (layer "F.Cu") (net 12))
 (segment (start 104 56.25) (end 104 59.338478) (width 0.2) (layer "F.Cu") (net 12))
 (segment (start 105 53.5) (end 102.623736 55.876264) (width 0.2) (layer "F.Cu") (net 11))
 (segment (start 102.623736 55.876264) (end 101.457025 55.876264) (width 0.2) (layer "F.Cu") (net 11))
 (segment (start 101.457025 55.876264) (end 100.992194 55.411433) (width 0.2) (layer "F.Cu") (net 11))
 (segment (start 108.8875 53.5) (end 105 53.5) (width 0.2) (layer "F.Cu") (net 11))
 (segment (start 102.282664 62.217336) (end 91.75 62.217336) (width 0.2) (layer "F.Cu") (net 19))
 (segment (start 134.7885 68.7115) (end 134 69.5) (width 0.2) (layer "F.Cu") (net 51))
 (segment (start 134.7885 61.109676) (end 134.7885 68.7115) (width 0.2) (layer "F.Cu") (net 51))
 (segment (start 132.428824 58.75) (end 134.7885 61.109676) (width 0.2) (layer "F.Cu") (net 51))
 (segment (start 131.82 58.75) (end 132.428824 58.75) (width 0.2) (layer "F.Cu") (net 51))
 (segment (start 132.428824 61.75) (end 131.82 61.75) (width 0.2) (layer "F.Cu") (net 42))
 (segment (start 134 68) (end 134 63.321176) (width 0.2) (layer "F.Cu") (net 42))
 (segment (start 134 63.321176) (end 132.428824 61.75) (width 0.2) (layer "F.Cu") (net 42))
 (segment (start 116.5 53) (end 121.725 58.225) (width 0.2) (layer "F.Cu") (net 6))
 (segment (start 121.725 58.225) (end 124.3625 58.225) (width 0.2) (layer "F.Cu") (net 6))
 (segment (start 113.1125 53) (end 116.5 53) (width 0.2) (layer "F.Cu") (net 6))
 (segment (start 132.175 68) (end 132.175 69.5) (width 0.2) (layer "F.Cu") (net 1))
 (segment (start 131.82 57.3) (end 126.59487 57.3) (width 0.2) (layer "F.Cu") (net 1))
 (segment (start 126.59487 57.3) (end 125.01987 58.875) (width 0.2) (layer "F.Cu") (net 1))
 (segment (start 125.01987 58.875) (end 124.3625 58.875) (width 0.2) (layer "F.Cu") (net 1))
 (segment (start 113.146447 58) (end 111.994976 59.151471) (width 0.2) (layer "F.Cu") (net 7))
 (segment (start 116.9421 58.875) (end 116.0671 58) (width 0.2) (layer "F.Cu") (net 7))
 (segment (start 118.6375 58.875) (end 116.9421 58.875) (width 0.2) (layer "F.Cu") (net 7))
 (segment (start 116.0671 58) (end 113.146447 58) (width 0.2) (layer "F.Cu") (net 7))
 (segment (start 117.025 59.525) (end 116 58.5) (width 0.2) (layer "F.Cu") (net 8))
 (segment (start 116 58.5) (end 113.353553 58.5) (width 0.2) (layer "F.Cu") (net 8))
 (segment (start 113.353553 58.5) (end 112.348529 59.505024) (width 0.2) (layer "F.Cu") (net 8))
 (segment (start 118.6375 59.525) (end 117.025 59.525) (width 0.2) (layer "F.Cu") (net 8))
 (segment (start 112.290388 61.780335) (end 111.994976 61.484923) (width 0.2) (layer "F.Cu") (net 29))
 (segment (start 115.7421 60.825) (end 114.786765 61.780335) (width 0.2) (layer "F.Cu") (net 29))
 (segment (start 118.6375 60.825) (end 115.7421 60.825) (width 0.2) (layer "F.Cu") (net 29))
 (segment (start 114.786765 61.780335) (end 112.290388 61.780335) (width 0.2) (layer "F.Cu") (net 29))
 (segment (start 112.596494 61.379335) (end 114.620665 61.379335) (width 0.2) (layer "F.Cu") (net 28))
 (segment (start 112.348529 61.13137) (end 112.596494 61.379335) (width 0.2) (layer "F.Cu") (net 28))
 (segment (start 115.825 60.175) (end 118.6375 60.175) (width 0.2) (layer "F.Cu") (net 28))
 (segment (start 114.620665 61.379335) (end 115.825 60.175) (width 0.2) (layer "F.Cu") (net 28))
 (segment (start 112.702083 59.858578) (end 113.060661 59.5) (width 0.2) (layer "F.Cu") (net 32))
 (segment (start 113.060661 59.5) (end 114.5 59.5) (width 0.2) (layer "F.Cu") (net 32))
 (segment (start 118.4885 62.626) (end 116.874 62.626) (width 0.2) (layer "F.Cu") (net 32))
 (segment (start 116.5 63) (end 116 63) (width 0.2) (layer "F.Cu") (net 32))
 (segment (start 118.6375 62.775) (end 118.4885 62.626) (width 0.2) (layer "F.Cu") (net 32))
 (segment (start 116.874 62.626) (end 116.5 63) (width 0.2) (layer "F.Cu") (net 32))
 (via (at 114.5 59.5) (size 0.6) (drill 0.3) (layers "F.Cu" "B.Cu") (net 32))
 (via (at 116 63) (size 0.6) (drill 0.3) (layers "F.Cu" "B.Cu") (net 32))
 (segment (start 114.5 59.5) (end 115.5 60.5) (width 0.2) (layer "B.Cu") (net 32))
 (segment (start 115.5 62.5) (end 116 63) (width 0.2) (layer "B.Cu") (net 32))
 (segment (start 115.5 60.5) (end 115.5 62.5) (width 0.2) (layer "B.Cu") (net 32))
 (segment (start 118.581165 62.181335) (end 118.6375 62.125) (width 0.2) (layer "F.Cu") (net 31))
 (segment (start 111.98428 62.181335) (end 118.581165 62.181335) (width 0.2) (layer "F.Cu") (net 31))
 (segment (start 111.641422 61.838477) (end 111.98428 62.181335) (width 0.2) (layer "F.Cu") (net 31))
 (segment (start 107.512782 62.478179) (end 107.034603 62) (width 0.2) (layer "F.Cu") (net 22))
 (segment (start 104.823044 62) (end 103.661522 60.838478) (width 0.2) (layer "F.Cu") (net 22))
 (segment (start 109.5 63.060661) (end 110.722184 61.838477) (width 0.2) (layer "F.Cu") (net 22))
 (segment (start 107.512782 62.487218) (end 107.5 62.5) (width 0.2) (layer "F.Cu") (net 22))
 (segment (start 107.512782 62.478179) (end 107.512782 62.487218) (width 0.2) (layer "F.Cu") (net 22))
 (segment (start 107.034603 62) (end 104.823044 62) (width 0.2) (layer "F.Cu") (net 22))
 (segment (start 109.5 63.202082) (end 109.5 63.060661) (width 0.2) (layer "F.Cu") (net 22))
 (segment (start 108.868342 63.83374) (end 109.5 63.202082) (width 0.2) (layer "F.Cu") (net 22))
 (via (at 107.512782 62.478179) (size 0.6) (drill 0.3) (layers "F.Cu" "B.Cu") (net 22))
 (via (at 108.868342 63.83374) (size 0.6) (drill 0.3) (layers "F.Cu" "B.Cu") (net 22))
 (segment (start 108.868342 63.83374) (end 107.512782 62.478179) (width 0.2) (layer "B.Cu") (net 22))
 (segment (start 103.201903 61.298097) (end 105.153806 63.25) (width 0.2) (layer "F.Cu") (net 21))
 (segment (start 108.603553 63.25) (end 110.36863 61.484923) (width 0.2) (layer "F.Cu") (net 21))
 (segment (start 105.153806 63.25) (end 108.603553 63.25) (width 0.2) (layer "F.Cu") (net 21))
 (segment (start 109.646447 61.5) (end 105.242284 61.5) (width 0.2) (layer "F.Cu") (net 23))
 (segment (start 105.242284 61.5) (end 104.121142 60.378858) (width 0.2) (layer "F.Cu") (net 23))
 (segment (start 110.015077 61.13137) (end 109.646447 61.5) (width 0.2) (layer "F.Cu") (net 23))
 (segment (start 107.990428 60.990428) (end 109.448911 60.990428) (width 0.2) (layer "F.Cu") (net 20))
 (segment (start 107.5 60.5) (end 107.990428 60.990428) (width 0.2) (layer "F.Cu") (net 20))
 (segment (start 109.448911 60.990428) (end 109.661523 60.777816) (width 0.2) (layer "F.Cu") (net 20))
 (segment (start 103.984567 63) (end 102.742284 61.757717) (width 0.2) (layer "F.Cu") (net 20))
 (via (at 107.5 60.5) (size 0.6) (drill 0.3) (layers "F.Cu" "B.Cu") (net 20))
 (via (at 103.984567 63) (size 0.6) (drill 0.3) (layers "F.Cu" "B.Cu") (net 20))
 (segment (start 103.984567 63) (end 105 63) (width 0.2) (layer "B.Cu") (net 20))
 (segment (start 105 63) (end 107.5 60.5) (width 0.2) (layer "B.Cu") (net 20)))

